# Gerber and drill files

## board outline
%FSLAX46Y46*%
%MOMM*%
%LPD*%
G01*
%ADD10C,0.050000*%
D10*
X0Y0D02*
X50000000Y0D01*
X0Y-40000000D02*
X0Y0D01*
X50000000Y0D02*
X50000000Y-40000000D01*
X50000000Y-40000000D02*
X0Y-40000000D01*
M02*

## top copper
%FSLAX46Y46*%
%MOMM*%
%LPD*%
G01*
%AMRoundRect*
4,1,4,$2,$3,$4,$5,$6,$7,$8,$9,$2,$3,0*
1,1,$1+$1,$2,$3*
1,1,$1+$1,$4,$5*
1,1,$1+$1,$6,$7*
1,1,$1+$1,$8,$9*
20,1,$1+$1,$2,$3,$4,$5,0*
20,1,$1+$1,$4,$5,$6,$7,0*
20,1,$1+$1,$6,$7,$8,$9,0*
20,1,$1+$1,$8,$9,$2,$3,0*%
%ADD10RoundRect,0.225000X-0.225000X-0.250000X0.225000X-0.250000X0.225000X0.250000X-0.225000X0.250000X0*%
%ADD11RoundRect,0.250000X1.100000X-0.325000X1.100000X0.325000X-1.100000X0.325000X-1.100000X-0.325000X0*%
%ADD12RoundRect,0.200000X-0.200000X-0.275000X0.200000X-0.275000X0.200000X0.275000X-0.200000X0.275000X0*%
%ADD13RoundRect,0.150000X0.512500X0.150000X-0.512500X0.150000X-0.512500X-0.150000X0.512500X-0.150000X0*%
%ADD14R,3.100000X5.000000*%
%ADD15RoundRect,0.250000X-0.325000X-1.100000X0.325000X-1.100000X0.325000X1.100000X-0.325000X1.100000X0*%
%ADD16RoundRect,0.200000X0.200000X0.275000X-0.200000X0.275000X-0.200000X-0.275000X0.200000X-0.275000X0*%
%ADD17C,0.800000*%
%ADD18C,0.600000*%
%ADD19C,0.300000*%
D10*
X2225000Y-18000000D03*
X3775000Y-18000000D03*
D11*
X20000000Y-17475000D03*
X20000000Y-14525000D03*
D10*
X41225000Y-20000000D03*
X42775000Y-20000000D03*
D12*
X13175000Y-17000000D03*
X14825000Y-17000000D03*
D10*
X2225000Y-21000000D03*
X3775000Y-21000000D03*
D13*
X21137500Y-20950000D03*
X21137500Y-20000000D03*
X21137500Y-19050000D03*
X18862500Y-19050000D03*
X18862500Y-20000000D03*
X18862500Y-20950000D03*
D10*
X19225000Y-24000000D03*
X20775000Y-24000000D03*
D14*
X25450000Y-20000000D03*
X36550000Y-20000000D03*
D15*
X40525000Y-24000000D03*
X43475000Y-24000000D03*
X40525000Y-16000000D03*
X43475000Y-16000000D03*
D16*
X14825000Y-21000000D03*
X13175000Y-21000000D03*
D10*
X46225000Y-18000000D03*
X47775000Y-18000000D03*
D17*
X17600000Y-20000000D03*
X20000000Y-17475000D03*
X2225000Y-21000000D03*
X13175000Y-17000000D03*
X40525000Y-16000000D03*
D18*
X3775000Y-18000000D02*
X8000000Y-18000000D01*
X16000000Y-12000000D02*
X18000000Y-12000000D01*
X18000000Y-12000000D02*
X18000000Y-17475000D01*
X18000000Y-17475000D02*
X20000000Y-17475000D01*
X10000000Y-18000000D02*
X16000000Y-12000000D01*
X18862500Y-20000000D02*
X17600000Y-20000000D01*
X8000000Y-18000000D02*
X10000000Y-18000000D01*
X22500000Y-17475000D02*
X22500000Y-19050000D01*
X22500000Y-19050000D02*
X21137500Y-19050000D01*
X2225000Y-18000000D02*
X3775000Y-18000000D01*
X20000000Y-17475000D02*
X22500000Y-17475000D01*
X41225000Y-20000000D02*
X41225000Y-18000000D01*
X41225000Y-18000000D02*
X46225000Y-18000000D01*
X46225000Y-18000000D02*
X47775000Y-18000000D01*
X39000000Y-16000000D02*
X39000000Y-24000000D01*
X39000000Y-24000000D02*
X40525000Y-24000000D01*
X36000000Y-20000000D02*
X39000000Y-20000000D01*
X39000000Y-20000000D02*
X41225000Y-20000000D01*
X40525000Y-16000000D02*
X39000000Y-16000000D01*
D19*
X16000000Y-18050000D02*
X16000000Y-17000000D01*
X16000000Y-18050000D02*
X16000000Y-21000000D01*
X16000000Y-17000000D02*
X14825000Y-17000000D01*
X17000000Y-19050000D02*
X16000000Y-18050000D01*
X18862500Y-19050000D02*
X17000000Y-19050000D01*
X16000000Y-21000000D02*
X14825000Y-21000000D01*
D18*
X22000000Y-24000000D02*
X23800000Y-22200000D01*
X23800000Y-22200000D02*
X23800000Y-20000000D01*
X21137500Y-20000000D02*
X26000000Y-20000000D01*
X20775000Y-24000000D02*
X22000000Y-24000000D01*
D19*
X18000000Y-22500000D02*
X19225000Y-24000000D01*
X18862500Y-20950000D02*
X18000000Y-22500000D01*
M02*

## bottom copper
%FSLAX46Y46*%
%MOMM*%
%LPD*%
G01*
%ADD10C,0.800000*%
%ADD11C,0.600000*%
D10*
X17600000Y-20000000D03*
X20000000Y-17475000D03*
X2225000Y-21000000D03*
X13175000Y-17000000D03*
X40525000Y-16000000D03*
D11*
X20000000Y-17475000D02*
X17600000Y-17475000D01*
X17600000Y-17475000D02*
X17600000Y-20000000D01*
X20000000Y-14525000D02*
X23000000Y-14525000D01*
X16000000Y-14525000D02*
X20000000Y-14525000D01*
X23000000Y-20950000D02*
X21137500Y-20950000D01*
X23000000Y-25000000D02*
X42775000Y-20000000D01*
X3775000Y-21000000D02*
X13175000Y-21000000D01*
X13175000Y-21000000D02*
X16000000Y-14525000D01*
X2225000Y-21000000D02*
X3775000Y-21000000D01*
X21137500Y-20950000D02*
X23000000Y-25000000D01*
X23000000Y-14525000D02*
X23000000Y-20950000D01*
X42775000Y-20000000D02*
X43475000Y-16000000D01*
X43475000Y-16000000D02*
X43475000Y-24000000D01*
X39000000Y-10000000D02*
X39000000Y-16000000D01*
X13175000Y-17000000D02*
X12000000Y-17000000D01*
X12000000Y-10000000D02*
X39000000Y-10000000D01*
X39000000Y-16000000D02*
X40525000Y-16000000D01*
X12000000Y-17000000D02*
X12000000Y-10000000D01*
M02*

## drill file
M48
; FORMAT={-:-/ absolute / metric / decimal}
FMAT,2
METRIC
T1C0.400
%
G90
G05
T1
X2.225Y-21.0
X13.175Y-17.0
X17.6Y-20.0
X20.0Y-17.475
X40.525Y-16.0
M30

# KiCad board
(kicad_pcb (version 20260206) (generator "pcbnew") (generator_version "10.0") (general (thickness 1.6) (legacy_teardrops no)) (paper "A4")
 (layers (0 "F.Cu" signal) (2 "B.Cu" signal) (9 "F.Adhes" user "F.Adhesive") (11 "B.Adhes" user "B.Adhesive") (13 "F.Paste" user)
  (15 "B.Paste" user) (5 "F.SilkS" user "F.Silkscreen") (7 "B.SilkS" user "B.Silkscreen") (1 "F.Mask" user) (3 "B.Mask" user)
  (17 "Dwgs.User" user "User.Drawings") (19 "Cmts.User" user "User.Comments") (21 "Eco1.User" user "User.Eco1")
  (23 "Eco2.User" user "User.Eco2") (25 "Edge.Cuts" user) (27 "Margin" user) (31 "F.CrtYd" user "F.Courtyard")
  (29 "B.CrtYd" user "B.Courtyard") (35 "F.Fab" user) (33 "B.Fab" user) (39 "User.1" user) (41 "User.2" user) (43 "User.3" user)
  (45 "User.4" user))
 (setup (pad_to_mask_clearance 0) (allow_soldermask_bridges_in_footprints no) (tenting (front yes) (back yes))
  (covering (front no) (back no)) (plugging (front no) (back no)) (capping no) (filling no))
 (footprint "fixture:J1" (layer "F.Cu") (at 3 18)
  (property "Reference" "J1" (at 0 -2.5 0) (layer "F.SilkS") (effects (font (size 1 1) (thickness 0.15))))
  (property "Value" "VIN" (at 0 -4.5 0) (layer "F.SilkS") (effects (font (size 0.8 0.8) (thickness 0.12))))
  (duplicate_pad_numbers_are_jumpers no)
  (pad "1" smd roundrect (at -0.775 0) (size 0.9 0.95) (layers "F.Cu" "F.Mask" "F.Paste") (roundrect_rratio 0.25) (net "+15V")
   (thermal_bridge_angle 45))
  (pad "2" smd roundrect (at 0.775 0) (size 0.9 0.95) (layers "F.Cu" "F.Mask" "F.Paste") (roundrect_rratio 0.25) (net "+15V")
   (thermal_bridge_angle 45)))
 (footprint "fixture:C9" (layer "F.Cu") (at 20 16 90)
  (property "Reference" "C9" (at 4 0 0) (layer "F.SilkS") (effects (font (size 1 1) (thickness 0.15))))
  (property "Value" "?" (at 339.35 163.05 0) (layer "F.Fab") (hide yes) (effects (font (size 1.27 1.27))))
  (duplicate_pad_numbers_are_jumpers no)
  (pad "1" smd roundrect (at -1.475 0 90) (size 1.15 2.7) (layers "F.Cu" "F.Mask" "F.Paste") (roundrect_rratio 0.217391) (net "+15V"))
  (pad "2" smd roundrect (at 1.475 0 90) (size 1.15 2.7) (layers "F.Cu" "F.Mask" "F.Paste") (roundrect_rratio 0.217391) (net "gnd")))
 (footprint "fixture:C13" (layer "F.Cu") (at 42 20)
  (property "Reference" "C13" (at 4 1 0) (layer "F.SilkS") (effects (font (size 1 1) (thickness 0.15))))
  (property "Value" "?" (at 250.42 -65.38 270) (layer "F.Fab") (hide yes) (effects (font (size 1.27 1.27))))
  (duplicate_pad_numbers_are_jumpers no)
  (pad "1" smd roundrect (at -0.775 0) (size 0.9 0.95) (layers "F.Cu" "F.Mask" "F.Paste") (roundrect_rratio 0.25) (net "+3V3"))
  (pad "2" smd roundrect (at 0.775 0) (size 0.9 0.95) (layers "F.Cu" "F.Mask" "F.Paste") (roundrect_rratio 0.25) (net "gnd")))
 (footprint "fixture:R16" (layer "F.Cu") (at 14 17)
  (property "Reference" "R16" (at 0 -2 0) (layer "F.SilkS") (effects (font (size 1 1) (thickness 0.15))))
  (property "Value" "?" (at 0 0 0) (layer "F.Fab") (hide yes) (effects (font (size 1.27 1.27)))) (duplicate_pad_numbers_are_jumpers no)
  (pad "1" smd roundrect (at -0.825 0) (size 0.8 0.95) (layers "F.Cu" "F.Mask" "F.Paste") (roundrect_rratio 0.25) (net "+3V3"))
  (pad "2" smd roundrect (at 0.825 0) (size 0.8 0.95) (layers "F.Cu" "F.Mask" "F.Paste") (roundrect_rratio 0.25) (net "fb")))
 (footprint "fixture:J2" (layer "F.Cu") (at 3 21)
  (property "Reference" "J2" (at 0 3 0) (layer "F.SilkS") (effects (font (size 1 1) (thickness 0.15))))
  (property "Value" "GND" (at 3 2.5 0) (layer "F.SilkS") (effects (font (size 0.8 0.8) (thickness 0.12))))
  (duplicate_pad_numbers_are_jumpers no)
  (pad "1" smd roundrect (at -0.775 0) (size 0.9 0.95) (layers "F.Cu" "F.Mask" "F.Paste") (roundrect_rratio 0.25) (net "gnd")
   (thermal_bridge_angle 45))
  (pad "2" smd roundrect (at 0.775 0) (size 0.9 0.95) (layers "F.Cu" "F.Mask" "F.Paste") (roundrect_rratio 0.25) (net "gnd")
   (thermal_bridge_angle 45)))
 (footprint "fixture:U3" (layer "F.Cu") (at 20 20 180)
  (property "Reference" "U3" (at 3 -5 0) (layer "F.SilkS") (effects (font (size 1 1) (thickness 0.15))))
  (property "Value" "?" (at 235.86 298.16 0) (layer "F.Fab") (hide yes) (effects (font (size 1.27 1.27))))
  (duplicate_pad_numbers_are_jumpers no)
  (pad "1" smd roundrect (at -1.1375 -0.95 180) (size 1.325 0.6) (layers "F.Cu" "F.Mask" "F.Paste") (roundrect_rratio 0.25) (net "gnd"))
  (pad "2" smd roundrect (at -1.1375 0 180) (size 1.325 0.6) (layers "F.Cu" "F.Mask" "F.Paste") (roundrect_rratio 0.25) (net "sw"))
  (pad "3" smd roundrect (at -1.1375 0.95 180) (size 1.325 0.6) (layers "F.Cu" "F.Mask" "F.Paste") (roundrect_rratio 0.25) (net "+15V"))
  (pad "4" smd roundrect (at 1.1375 0.95 180) (size 1.325 0.6) (layers "F.Cu" "F.Mask" "F.Paste") (roundrect_rratio 0.25) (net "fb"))
  (pad "5" smd roundrect (at 1.1375 0 180) (size 1.325 0.6) (layers "F.Cu" "F.Mask" "F.Paste") (roundrect_rratio 0.25) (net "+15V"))
  (pad "6" smd roundrect (at 1.1375 -0.95 180) (size 1.325 0.6) (layers "F.Cu" "F.Mask" "F.Paste") (roundrect_rratio 0.25) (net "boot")))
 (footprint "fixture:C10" (layer "F.Cu") (at 20 24)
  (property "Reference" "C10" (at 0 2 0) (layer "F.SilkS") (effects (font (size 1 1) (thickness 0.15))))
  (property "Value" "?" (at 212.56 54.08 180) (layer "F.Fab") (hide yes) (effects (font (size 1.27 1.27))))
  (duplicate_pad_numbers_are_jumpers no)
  (pad "1" smd roundrect (at -0.775 0) (size 0.9 0.95) (layers "F.Cu" "F.Mask" "F.Paste") (roundrect_rratio 0.25) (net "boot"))
  (pad "2" smd roundrect (at 0.775 0) (size 0.9 0.95) (layers "F.Cu" "F.Mask" "F.Paste") (roundrect_rratio 0.25) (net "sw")))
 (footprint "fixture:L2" (layer "F.Cu") (at 31 20)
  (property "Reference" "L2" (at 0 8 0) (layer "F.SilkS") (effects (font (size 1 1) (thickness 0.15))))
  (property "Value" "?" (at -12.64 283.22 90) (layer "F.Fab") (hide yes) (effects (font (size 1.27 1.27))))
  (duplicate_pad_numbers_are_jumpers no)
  (pad "1" smd rect (at -5.55 0) (size 3.1 5) (layers "F.Cu" "F.Mask" "F.Paste") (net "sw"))
  (pad "2" smd rect (at 5.55 0) (size 3.1 5) (layers "F.Cu" "F.Mask" "F.Paste") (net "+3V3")))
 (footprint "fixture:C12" (layer "F.Cu") (at 42 24)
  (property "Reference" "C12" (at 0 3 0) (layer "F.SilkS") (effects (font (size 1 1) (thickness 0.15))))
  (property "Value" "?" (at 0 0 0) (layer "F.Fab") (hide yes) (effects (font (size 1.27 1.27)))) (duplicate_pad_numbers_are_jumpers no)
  (pad "1" smd roundrect (at -1.475 0) (size 1.15 2.7) (layers "F.Cu" "F.Mask" "F.Paste") (roundrect_rratio 0.217391) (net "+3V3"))
  (pad "2" smd roundrect (at 1.475 0) (size 1.15 2.7) (layers "F.Cu" "F.Mask" "F.Paste") (roundrect_rratio 0.217391) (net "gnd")))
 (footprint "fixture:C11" (layer "F.Cu") (at 42 16)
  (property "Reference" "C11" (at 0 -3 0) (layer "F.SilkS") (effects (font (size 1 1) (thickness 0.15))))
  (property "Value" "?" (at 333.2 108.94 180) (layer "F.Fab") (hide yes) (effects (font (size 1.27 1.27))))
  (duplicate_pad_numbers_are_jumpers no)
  (pad "1" smd roundrect (at -1.475 0) (size 1.15 2.7) (layers "F.Cu" "F.Mask" "F.Paste") (roundrect_rratio 0.217391) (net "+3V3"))
  (pad "2" smd roundrect (at 1.475 0) (size 1.15 2.7) (layers "F.Cu" "F.Mask" "F.Paste") (roundrect_rratio 0.217391) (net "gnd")))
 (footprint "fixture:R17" (layer "F.Cu") (at 14 21 180)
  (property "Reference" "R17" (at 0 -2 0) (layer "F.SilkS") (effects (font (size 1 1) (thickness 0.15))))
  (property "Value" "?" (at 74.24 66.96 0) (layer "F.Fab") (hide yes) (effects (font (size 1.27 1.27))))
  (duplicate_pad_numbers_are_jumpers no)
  (pad "1" smd roundrect (at -0.825 0 180) (size 0.8 0.95) (layers "F.Cu" "F.Mask" "F.Paste") (roundrect_rratio 0.25) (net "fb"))
  (pad "2" smd roundrect (at 0.825 0 180) (size 0.8 0.95) (layers "F.Cu" "F.Mask" "F.Paste") (roundrect_rratio 0.25) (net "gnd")))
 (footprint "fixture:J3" (layer "F.Cu") (at 47 18)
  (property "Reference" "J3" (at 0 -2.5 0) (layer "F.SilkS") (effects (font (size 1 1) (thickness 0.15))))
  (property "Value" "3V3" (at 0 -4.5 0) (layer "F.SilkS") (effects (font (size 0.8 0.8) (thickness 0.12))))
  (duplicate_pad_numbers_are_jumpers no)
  (pad "1" smd roundrect (at -0.775 0) (size 0.9 0.95) (layers "F.Cu" "F.Mask" "F.Paste") (roundrect_rratio 0.25) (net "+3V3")
   (thermal_bridge_angle 45))
  (pad "2" smd roundrect (at 0.775 0) (size 0.9 0.95) (layers "F.Cu" "F.Mask" "F.Paste") (roundrect_rratio 0.25) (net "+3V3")
   (thermal_bridge_angle 45)))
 (gr_line (start 0 0) (end 50 0) (stroke (width 0.05) (type default)) (layer "Edge.Cuts"))
 (gr_line (start 0 40) (end 0 0) (stroke (width 0.05) (type default)) (layer "Edge.Cuts"))
 (gr_line (start 50 0) (end 50 40) (stroke (width 0.05) (type default)) (layer "Edge.Cuts"))
 (gr_line (start 50 40) (end 0 40) (stroke (width 0.05) (type default)) (layer "Edge.Cuts"))
 (segment (start 3.775 18) (end 8 18) (width 0.6) (layer "F.Cu") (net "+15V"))
 (segment (start 16 12) (end 18 12) (width 0.6) (layer "F.Cu") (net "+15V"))
 (segment (start 18 12) (end 18 17.475) (width 0.6) (layer "F.Cu") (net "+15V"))
 (segment (start 18 17.475) (end 20 17.475) (width 0.6) (layer "F.Cu") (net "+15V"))
 (segment (start 10 18) (end 16 12) (width 0.6) (layer "F.Cu") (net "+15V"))
 (segment (start 18.8625 20) (end 17.6 20) (width 0.6) (layer "F.Cu") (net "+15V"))
 (segment (start 8 18) (end 10 18) (width 0.6) (layer "F.Cu") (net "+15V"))
 (segment (start 22.5 17.475) (end 22.5 19.05) (width 0.6) (layer "F.Cu") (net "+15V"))
 (segment (start 22.5 19.05) (end 21.1375 19.05) (width 0.6) (layer "F.Cu") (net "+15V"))
 (segment (start 2.225 18) (end 3.775 18) (width 0.6) (layer "F.Cu") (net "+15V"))
 (segment (start 20 17.475) (end 22.5 17.475) (width 0.6) (layer "F.Cu") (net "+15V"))
 (via (at 17.6 20) (size 0.8) (drill 0.4) (layers "F.Cu" "B.Cu") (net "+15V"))
 (via (at 20 17.475) (size 0.8) (drill 0.4) (layers "F.Cu" "B.Cu") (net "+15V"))
 (segment (start 20 17.475) (end 17.6 17.475) (width 0.6) (layer "B.Cu") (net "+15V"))
 (segment (start 17.6 17.475) (end 17.6 20) (width 0.6) (layer "B.Cu") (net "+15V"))
 (via (at 2.225 21) (size 0.8) (drill 0.4) (layers "F.Cu" "B.Cu") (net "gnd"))
 (segment (start 20 14.525) (end 23 14.525) (width 0.6) (layer "B.Cu") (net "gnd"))
 (segment (start 16 14.525) (end 20 14.525) (width 0.6) (layer "B.Cu") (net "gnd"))
 (segment (start 23 20.95) (end 21.1375 20.95) (width 0.6) (layer "B.Cu") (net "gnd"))
 (segment (start 23 25) (end 42.775 20) (width 0.6) (layer "B.Cu") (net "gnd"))
 (segment (start 3.775 21) (end 13.175 21) (width 0.6) (layer "B.Cu") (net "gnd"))
 (segment (start 13.175 21) (end 16 14.525) (width 0.6) (layer "B.Cu") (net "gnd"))
 (segment (start 2.225 21) (end 3.775 21) (width 0.6) (layer "B.Cu") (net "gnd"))
 (segment (start 21.1375 20.95) (end 23 25) (width 0.6) (layer "B.Cu") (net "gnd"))
 (segment (start 23 14.525) (end 23 20.95) (width 0.6) (layer "B.Cu") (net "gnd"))
 (segment (start 42.775 20) (end 43.475 16) (width 0.6) (layer "B.Cu") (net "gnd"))
 (segment (start 43.475 16) (end 43.475 24) (width 0.6) (layer "B.Cu") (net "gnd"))
 (segment (start 41.225 20) (end 41.225 18) (width 0.6) (layer "F.Cu") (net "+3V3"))
 (segment (start 41.225 18) (end 46.225 18) (width 0.6) (layer "F.Cu") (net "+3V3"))
 (segment (start 46.225 18) (end 47.775 18) (width 0.6) (layer "F.Cu") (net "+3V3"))
 (segment (start 39 16) (end 39 24) (width 0.6) (layer "F.Cu") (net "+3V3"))
 (segment (start 39 24) (end 40.525 24) (width 0.6) (layer "F.Cu") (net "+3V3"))
 (segment (start 36 20) (end 39 20) (width 0.6) (layer "F.Cu") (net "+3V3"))
 (segment (start 39 20) (end 41.225 20) (width 0.6) (layer "F.Cu") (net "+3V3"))
 (segment (start 40.525 16) (end 39 16) (width 0.6) (layer "F.Cu") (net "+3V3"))
 (via (at 13.175 17) (size 0.8) (drill 0.4) (layers "F.Cu" "B.Cu") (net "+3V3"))
 (via (at 40.525 16) (size 0.8) (drill 0.4) (layers "F.Cu" "B.Cu") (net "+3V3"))
 (segment (start 39 10) (end 39 16) (width 0.6) (layer "B.Cu") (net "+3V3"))
 (segment (start 13.175 17) (end 12 17) (width 0.6) (layer "B.Cu") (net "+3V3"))
 (segment (start 12 10) (end 39 10) (width 0.6) (layer "B.Cu") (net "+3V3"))
 (segment (start 39 16) (end 40.525 16) (width 0.6) (layer "B.Cu") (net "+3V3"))
 (segment (start 12 17) (end 12 10) (width 0.6) (layer "B.Cu") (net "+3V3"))
 (segment (start 16 18.05) (end 16 17) (width 0.3) (layer "F.Cu") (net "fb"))
 (segment (start 16 18.05) (end 16 21) (width 0.3) (layer "F.Cu") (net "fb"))
 (segment (start 16 17) (end 14.825 17) (width 0.3) (layer "F.Cu") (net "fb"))
 (segment (start 17 19.05) (end 16 18.05) (width 0.3) (layer "F.Cu") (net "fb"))
 (segment (start 18.8625 19.05) (end 17 19.05) (width 0.3) (layer "F.Cu") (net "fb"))
 (segment (start 16 21) (end 14.825 21) (width 0.3) (layer "F.Cu") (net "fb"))
 (segment (start 22 24) (end 23.8 22.2) (width 0.6) (layer "F.Cu") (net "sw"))
 (segment (start 23.8 22.2) (end 23.8 20) (width 0.6) (layer "F.Cu") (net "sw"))
 (segment (start 21.1375 20) (end 26 20) (width 0.6) (layer "F.Cu") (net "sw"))
 (segment (start 20.775 24) (end 22 24) (width 0.6) (layer "F.Cu") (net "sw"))
 (segment (start 18 22.5) (end 19.225 24) (width 0.3) (layer "F.Cu") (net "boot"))
 (segment (start 18.8625 20.95) (end 18 22.5) (width 0.3) (layer "F.Cu") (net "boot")))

